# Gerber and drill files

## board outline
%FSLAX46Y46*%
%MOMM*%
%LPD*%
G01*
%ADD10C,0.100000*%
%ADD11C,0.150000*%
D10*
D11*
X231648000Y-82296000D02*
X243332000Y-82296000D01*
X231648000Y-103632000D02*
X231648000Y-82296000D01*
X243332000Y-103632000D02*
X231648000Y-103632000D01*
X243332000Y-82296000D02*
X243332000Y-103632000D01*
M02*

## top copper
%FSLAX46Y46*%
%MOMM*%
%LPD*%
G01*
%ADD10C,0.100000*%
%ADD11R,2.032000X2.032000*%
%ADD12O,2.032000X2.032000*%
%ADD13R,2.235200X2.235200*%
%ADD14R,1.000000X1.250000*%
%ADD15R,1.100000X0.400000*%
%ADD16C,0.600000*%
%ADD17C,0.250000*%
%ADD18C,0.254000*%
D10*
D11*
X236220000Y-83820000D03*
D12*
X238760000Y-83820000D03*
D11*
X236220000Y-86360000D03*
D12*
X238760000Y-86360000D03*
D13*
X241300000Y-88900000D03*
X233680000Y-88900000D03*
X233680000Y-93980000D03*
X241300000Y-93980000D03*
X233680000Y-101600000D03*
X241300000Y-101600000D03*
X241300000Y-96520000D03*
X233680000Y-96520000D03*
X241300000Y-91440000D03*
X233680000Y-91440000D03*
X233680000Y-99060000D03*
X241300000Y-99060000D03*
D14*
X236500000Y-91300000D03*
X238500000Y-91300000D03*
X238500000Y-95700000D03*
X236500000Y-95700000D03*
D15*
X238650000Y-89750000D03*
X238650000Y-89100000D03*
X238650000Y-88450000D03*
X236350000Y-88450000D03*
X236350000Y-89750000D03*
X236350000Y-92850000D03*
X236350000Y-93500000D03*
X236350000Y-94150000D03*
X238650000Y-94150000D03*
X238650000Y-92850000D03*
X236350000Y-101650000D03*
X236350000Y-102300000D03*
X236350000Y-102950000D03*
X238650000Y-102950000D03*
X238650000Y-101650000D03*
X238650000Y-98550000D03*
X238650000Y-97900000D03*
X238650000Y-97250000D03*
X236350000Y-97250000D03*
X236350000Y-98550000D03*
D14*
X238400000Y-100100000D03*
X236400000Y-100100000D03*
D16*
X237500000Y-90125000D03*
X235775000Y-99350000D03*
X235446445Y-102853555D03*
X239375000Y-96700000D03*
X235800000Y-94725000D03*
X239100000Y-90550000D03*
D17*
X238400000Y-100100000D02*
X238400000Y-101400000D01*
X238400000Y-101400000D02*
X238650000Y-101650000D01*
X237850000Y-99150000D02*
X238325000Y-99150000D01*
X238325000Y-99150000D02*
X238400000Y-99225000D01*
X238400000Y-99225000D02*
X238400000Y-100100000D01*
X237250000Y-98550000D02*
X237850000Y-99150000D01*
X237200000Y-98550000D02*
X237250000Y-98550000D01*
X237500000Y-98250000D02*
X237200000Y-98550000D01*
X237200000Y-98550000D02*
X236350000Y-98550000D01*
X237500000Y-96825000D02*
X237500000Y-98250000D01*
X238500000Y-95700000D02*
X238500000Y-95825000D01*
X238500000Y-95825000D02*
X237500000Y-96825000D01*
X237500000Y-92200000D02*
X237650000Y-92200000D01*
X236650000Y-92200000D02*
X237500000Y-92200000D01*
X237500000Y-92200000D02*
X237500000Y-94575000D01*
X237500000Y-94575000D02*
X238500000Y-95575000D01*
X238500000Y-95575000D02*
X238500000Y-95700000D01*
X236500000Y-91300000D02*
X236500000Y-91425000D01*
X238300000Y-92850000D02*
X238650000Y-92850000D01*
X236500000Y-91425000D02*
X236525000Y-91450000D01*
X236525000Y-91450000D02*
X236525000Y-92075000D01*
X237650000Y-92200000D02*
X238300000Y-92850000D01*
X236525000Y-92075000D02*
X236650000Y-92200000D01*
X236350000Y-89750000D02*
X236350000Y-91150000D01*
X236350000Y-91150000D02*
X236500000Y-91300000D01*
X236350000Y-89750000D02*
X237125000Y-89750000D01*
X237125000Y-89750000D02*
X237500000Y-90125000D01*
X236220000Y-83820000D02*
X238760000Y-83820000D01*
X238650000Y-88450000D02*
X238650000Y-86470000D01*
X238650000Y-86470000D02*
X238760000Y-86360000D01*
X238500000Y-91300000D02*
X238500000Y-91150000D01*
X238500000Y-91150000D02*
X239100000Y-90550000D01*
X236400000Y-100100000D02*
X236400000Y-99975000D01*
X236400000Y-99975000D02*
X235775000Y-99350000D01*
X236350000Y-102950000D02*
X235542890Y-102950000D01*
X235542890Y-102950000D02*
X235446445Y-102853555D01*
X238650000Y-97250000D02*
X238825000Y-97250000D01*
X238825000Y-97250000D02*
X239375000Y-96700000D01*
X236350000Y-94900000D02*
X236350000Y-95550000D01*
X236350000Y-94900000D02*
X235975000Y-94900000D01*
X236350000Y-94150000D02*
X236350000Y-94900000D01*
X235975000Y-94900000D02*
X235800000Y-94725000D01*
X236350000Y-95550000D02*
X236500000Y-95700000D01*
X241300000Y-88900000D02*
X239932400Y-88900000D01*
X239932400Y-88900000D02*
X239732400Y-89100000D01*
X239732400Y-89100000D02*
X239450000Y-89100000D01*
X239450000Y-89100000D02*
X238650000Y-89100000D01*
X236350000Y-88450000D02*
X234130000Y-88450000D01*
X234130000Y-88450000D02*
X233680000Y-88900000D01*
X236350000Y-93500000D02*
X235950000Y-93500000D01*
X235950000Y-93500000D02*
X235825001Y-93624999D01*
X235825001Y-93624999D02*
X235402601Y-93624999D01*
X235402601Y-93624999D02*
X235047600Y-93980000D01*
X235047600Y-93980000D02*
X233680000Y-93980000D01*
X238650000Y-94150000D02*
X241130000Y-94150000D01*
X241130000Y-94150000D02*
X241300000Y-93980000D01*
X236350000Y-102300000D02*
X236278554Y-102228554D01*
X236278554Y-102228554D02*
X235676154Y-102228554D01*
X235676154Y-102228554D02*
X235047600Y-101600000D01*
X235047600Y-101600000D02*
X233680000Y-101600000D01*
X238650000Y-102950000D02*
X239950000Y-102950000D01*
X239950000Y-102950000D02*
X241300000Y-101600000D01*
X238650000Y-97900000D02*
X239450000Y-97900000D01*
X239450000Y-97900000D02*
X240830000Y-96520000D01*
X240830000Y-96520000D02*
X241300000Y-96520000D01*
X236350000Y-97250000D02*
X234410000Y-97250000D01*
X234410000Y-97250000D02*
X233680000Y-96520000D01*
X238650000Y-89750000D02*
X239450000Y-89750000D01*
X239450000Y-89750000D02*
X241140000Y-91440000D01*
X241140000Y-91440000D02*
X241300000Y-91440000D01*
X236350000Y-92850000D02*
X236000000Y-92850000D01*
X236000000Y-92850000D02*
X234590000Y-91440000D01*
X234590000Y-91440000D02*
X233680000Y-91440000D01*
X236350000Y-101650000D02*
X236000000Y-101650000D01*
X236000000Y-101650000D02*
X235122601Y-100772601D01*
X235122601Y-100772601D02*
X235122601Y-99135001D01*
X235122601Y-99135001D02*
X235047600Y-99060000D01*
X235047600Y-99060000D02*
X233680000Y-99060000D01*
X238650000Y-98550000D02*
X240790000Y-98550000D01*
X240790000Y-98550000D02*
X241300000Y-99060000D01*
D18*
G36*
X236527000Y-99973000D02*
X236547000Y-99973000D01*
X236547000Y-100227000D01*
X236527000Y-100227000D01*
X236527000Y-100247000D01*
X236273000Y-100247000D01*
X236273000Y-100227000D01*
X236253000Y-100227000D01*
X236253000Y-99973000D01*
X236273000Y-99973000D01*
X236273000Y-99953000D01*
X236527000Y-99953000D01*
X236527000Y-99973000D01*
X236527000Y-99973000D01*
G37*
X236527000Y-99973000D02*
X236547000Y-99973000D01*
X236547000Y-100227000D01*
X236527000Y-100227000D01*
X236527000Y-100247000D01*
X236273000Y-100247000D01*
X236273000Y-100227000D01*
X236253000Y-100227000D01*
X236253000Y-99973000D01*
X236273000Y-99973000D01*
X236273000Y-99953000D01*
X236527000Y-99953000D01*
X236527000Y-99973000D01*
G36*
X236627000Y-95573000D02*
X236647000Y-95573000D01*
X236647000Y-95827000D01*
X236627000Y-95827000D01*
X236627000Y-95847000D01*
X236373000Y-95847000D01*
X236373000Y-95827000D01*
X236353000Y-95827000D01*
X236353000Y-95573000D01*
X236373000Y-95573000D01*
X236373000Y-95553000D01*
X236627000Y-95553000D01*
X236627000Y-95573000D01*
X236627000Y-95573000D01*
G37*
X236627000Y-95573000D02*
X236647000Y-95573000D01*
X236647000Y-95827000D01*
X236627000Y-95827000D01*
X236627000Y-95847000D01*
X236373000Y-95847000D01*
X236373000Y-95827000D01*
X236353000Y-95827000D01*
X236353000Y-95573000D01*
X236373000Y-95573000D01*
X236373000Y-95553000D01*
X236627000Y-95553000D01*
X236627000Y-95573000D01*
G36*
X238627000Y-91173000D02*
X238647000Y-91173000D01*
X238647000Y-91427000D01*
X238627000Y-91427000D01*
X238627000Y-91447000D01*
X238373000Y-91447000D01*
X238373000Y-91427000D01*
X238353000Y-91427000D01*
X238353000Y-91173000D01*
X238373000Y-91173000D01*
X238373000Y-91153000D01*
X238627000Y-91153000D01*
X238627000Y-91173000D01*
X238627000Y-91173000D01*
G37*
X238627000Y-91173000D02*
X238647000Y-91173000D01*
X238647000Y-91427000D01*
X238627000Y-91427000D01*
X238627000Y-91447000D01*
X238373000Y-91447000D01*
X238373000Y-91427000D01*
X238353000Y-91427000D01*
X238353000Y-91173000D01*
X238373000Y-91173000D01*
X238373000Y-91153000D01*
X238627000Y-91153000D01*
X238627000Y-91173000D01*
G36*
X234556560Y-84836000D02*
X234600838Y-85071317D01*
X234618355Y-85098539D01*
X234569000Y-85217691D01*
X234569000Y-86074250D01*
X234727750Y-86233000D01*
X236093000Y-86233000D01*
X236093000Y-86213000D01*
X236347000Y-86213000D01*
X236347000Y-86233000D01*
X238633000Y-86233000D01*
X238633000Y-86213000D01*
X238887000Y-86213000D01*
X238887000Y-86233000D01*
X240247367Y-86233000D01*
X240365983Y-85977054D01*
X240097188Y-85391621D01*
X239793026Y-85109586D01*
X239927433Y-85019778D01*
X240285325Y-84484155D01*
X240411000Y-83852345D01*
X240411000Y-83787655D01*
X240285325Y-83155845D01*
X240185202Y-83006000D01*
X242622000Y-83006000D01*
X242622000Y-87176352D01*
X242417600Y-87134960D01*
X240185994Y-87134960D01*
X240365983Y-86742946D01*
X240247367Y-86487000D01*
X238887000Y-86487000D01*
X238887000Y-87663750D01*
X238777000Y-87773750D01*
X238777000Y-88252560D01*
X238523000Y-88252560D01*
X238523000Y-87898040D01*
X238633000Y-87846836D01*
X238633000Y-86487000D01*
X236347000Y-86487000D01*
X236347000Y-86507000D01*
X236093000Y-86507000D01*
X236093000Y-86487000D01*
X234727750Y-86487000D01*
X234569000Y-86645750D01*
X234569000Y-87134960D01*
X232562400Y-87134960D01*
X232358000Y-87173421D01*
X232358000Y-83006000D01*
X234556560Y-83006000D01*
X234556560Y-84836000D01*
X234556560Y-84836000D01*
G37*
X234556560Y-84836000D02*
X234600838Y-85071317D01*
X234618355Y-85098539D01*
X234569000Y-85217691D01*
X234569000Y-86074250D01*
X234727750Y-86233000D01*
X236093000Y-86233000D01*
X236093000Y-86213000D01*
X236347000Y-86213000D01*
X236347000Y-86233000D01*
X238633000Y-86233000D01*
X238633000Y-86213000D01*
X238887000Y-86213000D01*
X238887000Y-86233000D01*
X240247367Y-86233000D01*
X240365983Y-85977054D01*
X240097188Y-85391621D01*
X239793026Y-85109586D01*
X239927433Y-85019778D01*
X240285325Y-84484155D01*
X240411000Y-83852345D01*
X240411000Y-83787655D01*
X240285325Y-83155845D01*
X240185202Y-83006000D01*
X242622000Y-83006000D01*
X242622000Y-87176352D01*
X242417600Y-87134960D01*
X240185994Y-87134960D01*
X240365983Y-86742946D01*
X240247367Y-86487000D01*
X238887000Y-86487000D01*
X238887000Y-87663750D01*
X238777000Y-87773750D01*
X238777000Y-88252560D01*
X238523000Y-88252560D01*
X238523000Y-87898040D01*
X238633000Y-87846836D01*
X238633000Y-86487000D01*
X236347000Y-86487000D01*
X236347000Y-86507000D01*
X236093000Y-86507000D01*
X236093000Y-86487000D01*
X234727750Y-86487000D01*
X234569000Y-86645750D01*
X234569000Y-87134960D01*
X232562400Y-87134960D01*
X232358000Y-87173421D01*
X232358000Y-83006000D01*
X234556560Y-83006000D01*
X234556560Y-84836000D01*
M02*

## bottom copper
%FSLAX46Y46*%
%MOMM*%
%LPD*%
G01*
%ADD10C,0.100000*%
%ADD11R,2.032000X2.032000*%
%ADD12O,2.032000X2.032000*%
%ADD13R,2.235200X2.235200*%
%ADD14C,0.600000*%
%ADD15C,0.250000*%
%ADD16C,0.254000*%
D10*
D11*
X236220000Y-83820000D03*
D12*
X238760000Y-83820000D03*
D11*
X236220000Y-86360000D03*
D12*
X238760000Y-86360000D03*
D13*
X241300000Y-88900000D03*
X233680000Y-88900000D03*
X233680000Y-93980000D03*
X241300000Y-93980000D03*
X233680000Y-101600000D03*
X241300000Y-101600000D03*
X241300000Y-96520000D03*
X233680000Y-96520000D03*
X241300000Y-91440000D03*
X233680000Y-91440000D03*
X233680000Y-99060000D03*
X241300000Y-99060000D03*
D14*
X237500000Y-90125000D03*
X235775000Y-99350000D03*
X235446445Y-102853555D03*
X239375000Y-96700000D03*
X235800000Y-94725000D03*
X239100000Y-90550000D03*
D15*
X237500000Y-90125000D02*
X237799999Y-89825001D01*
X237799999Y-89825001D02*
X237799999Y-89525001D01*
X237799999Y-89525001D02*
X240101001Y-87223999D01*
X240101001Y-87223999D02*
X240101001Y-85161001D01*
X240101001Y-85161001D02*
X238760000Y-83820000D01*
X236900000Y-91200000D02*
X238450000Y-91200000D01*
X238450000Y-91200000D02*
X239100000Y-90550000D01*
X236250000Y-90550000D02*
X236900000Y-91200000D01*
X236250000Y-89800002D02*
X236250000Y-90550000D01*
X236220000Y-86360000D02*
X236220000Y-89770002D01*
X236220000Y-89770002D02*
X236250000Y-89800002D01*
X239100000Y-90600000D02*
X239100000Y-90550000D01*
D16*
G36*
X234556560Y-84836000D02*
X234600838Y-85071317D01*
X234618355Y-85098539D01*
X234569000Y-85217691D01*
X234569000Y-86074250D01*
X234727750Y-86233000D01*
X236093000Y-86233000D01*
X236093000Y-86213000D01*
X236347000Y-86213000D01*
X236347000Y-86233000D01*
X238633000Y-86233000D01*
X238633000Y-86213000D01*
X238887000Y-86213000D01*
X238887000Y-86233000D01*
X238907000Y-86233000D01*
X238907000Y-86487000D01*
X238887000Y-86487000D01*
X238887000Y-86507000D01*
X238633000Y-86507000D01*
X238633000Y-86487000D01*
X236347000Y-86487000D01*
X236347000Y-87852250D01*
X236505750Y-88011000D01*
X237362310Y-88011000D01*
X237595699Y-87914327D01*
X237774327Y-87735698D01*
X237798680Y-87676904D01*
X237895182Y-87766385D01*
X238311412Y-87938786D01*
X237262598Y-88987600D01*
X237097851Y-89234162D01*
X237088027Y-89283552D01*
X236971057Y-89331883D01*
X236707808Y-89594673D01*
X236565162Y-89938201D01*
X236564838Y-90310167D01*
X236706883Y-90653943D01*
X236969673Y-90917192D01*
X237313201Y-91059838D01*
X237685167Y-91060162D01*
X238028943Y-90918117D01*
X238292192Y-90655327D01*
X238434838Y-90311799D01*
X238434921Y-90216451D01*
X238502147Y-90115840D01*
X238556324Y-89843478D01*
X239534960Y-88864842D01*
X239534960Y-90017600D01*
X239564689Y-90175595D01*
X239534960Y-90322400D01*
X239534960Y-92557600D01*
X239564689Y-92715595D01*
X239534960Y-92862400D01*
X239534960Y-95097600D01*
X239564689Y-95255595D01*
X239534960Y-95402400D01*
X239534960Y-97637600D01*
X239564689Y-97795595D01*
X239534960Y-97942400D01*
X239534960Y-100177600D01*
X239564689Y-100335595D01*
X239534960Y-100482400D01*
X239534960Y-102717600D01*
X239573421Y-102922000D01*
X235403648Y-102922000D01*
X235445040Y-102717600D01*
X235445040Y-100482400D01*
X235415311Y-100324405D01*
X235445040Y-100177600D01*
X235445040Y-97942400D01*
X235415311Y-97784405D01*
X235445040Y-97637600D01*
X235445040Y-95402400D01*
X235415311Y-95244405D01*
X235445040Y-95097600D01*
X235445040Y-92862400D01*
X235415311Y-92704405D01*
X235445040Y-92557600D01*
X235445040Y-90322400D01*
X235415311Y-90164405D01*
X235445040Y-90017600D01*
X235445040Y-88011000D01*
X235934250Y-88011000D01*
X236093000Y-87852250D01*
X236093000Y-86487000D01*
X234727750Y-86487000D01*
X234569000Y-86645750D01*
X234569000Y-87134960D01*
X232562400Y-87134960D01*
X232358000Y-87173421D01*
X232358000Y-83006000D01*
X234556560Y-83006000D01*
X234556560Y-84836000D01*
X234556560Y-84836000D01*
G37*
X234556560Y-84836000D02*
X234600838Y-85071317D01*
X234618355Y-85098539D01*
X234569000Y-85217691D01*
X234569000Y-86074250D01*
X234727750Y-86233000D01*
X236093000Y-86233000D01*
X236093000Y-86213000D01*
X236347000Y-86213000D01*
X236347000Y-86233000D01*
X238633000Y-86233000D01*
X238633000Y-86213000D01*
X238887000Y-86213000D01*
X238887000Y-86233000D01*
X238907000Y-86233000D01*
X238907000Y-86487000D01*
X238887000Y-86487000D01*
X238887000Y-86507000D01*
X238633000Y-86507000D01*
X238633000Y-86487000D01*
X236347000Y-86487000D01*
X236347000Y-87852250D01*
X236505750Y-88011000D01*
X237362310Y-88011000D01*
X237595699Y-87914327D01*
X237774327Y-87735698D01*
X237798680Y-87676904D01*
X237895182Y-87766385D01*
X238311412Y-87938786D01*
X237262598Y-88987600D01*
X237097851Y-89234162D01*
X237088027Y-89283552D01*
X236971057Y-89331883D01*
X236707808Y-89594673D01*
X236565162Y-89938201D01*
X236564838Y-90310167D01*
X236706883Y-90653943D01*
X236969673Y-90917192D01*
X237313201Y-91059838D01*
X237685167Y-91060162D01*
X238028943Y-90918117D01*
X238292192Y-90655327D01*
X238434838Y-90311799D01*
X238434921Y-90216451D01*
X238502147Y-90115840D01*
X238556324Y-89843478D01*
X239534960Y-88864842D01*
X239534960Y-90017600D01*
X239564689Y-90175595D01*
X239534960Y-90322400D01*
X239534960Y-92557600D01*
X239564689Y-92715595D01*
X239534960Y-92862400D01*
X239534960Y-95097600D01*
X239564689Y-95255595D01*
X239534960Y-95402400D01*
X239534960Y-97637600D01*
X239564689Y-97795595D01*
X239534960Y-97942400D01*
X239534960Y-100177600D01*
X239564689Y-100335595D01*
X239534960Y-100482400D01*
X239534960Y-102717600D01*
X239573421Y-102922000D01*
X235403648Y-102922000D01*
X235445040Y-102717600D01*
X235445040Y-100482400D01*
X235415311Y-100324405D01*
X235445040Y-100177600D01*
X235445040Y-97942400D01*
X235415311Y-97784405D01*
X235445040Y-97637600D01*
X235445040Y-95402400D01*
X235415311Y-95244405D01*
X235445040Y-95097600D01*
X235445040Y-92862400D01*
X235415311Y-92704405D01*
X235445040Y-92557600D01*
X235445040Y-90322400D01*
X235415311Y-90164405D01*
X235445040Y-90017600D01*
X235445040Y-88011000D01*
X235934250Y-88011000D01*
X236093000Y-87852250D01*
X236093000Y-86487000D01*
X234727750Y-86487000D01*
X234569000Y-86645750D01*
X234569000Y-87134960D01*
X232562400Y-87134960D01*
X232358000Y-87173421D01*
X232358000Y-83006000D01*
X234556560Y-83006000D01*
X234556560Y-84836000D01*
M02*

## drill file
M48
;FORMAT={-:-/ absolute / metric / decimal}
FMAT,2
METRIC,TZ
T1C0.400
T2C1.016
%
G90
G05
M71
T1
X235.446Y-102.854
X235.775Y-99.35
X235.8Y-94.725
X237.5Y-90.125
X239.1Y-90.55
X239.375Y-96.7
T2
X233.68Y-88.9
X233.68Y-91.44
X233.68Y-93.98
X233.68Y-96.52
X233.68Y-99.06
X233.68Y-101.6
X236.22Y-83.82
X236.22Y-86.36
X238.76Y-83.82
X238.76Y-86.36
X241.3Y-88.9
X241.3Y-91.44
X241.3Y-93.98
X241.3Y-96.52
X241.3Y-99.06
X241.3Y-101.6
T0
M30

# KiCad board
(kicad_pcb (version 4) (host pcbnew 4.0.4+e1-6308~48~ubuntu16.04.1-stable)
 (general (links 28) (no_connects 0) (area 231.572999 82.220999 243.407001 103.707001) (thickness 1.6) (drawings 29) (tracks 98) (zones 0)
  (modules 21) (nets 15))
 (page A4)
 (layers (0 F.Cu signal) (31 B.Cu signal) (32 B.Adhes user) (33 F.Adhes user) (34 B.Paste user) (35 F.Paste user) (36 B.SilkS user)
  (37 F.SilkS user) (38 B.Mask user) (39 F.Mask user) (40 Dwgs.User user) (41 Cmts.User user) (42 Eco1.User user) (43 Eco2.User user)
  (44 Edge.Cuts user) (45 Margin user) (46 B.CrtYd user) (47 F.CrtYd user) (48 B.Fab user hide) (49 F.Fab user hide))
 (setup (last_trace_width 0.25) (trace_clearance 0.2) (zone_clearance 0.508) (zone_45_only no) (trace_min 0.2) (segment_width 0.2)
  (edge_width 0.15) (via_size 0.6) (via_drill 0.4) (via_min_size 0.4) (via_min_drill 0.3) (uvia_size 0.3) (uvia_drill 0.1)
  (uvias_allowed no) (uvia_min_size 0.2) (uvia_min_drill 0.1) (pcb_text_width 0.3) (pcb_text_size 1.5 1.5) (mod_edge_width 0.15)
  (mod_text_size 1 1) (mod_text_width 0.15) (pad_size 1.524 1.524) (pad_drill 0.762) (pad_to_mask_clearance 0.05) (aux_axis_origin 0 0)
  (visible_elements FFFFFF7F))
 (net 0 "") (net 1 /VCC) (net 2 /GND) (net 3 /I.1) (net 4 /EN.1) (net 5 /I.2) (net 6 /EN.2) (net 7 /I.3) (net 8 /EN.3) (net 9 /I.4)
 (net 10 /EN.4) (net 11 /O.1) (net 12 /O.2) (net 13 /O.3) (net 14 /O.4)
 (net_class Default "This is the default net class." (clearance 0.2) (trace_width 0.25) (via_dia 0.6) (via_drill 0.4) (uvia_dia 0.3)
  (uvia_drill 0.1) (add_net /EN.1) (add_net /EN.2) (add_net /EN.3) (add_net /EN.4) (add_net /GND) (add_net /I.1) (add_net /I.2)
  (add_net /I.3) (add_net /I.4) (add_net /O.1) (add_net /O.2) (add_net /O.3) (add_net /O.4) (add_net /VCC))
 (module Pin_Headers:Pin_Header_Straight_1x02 (layer F.Cu) (at 236.22 83.82 90)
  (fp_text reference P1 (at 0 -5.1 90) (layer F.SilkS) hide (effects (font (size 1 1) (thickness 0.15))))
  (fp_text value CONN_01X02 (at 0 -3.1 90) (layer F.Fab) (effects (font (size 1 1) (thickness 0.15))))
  (pad 1 thru_hole rect (at 0 0 90) (size 2.032 2.032) (drill 1.016) (layers *.Cu *.Mask F.SilkS) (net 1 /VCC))
  (pad 2 thru_hole oval (at 0 2.54 90) (size 2.032 2.032) (drill 1.016) (layers *.Cu *.Mask F.SilkS) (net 1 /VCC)))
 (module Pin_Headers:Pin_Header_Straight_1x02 (layer F.Cu) (at 236.22 86.36 90)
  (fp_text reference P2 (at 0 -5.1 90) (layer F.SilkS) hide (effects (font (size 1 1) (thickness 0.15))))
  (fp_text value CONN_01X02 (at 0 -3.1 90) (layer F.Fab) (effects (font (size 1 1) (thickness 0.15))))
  (pad 1 thru_hole rect (at 0 0 90) (size 2.032 2.032) (drill 1.016) (layers *.Cu *.Mask F.SilkS) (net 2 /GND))
  (pad 2 thru_hole oval (at 0 2.54 90) (size 2.032 2.032) (drill 1.016) (layers *.Cu *.Mask F.SilkS) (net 2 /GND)))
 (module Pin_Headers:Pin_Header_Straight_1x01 (layer F.Cu) (at 241.3 88.9 270)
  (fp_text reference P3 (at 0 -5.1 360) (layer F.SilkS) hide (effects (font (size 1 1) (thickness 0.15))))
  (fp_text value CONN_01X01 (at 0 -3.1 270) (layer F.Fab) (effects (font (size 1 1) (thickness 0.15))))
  (pad 1 thru_hole rect (at 0 0 270) (size 2.2352 2.2352) (drill 1.016) (layers *.Cu *.Mask F.SilkS) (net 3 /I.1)))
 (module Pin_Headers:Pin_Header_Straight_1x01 (layer F.Cu) (at 233.68 88.9 90)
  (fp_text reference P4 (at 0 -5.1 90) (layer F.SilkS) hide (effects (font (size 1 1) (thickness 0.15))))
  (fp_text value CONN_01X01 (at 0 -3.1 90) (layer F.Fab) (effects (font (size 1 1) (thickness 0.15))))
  (pad 1 thru_hole rect (at 0 0 90) (size 2.2352 2.2352) (drill 1.016) (layers *.Cu *.Mask F.SilkS) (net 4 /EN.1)))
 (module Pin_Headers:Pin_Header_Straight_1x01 (layer F.Cu) (at 233.68 93.98 90)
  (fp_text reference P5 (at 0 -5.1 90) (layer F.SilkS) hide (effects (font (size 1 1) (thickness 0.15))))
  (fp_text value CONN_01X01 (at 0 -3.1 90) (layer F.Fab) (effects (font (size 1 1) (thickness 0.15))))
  (pad 1 thru_hole rect (at 0 0 90) (size 2.2352 2.2352) (drill 1.016) (layers *.Cu *.Mask F.SilkS) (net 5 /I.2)))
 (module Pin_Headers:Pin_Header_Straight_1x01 (layer F.Cu) (at 241.3 93.98 270)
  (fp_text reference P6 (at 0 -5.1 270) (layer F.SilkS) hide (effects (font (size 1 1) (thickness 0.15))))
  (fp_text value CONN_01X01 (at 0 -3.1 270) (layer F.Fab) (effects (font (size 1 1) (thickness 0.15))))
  (pad 1 thru_hole rect (at 0 0 270) (size 2.2352 2.2352) (drill 1.016) (layers *.Cu *.Mask F.SilkS) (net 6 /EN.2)))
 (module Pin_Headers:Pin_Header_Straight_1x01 (layer F.Cu) (at 233.68 101.6 90)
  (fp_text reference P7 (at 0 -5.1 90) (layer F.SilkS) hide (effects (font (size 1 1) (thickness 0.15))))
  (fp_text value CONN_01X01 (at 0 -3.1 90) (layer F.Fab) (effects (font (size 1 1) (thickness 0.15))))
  (pad 1 thru_hole rect (at 0 0 90) (size 2.2352 2.2352) (drill 1.016) (layers *.Cu *.Mask F.SilkS) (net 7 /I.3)))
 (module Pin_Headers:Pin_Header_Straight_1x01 (layer F.Cu) (at 241.3 101.6 270)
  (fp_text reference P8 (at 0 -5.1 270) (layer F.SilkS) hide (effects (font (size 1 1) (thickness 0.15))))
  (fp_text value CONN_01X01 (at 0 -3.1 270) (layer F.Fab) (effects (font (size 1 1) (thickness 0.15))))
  (pad 1 thru_hole rect (at 0 0 270) (size 2.2352 2.2352) (drill 1.016) (layers *.Cu *.Mask F.SilkS) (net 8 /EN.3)))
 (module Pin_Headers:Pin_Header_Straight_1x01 (layer F.Cu) (at 241.3 96.52 270)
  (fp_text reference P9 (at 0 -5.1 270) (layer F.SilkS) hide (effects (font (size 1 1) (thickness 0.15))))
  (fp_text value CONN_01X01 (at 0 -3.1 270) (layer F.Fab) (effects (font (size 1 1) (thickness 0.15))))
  (pad 1 thru_hole rect (at 0 0 270) (size 2.2352 2.2352) (drill 1.016) (layers *.Cu *.Mask F.SilkS) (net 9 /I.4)))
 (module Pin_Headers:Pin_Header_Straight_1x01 (layer F.Cu) (at 233.68 96.52 90)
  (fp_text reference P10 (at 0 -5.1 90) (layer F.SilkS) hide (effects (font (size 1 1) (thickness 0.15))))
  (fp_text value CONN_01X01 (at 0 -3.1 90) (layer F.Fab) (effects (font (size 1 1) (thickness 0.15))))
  (pad 1 thru_hole rect (at 0 0 90) (size 2.2352 2.2352) (drill 1.016) (layers *.Cu *.Mask F.SilkS) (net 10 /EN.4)))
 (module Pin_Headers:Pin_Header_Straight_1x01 (layer F.Cu) (at 241.3 91.44 270)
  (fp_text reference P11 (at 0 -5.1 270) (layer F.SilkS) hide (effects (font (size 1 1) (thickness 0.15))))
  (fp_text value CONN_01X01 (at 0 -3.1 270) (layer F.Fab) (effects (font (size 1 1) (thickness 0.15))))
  (pad 1 thru_hole rect (at 0 0 270) (size 2.2352 2.2352) (drill 1.016) (layers *.Cu *.Mask F.SilkS) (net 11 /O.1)))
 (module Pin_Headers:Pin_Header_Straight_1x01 (layer F.Cu) (at 233.68 91.44 90)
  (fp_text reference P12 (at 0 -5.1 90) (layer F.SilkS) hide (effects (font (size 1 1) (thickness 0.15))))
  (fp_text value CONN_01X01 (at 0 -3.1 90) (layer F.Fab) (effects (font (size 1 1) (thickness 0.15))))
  (pad 1 thru_hole rect (at 0 0 90) (size 2.2352 2.2352) (drill 1.016) (layers *.Cu *.Mask F.SilkS) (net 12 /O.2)))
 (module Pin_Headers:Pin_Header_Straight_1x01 (layer F.Cu) (at 233.68 99.06 90)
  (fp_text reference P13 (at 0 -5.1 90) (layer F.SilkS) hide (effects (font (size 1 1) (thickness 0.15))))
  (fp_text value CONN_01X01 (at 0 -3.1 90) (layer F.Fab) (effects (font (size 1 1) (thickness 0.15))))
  (pad 1 thru_hole rect (at 0 0 90) (size 2.2352 2.2352) (drill 1.016) (layers *.Cu *.Mask F.SilkS) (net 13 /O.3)))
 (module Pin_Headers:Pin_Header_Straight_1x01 (layer F.Cu) (at 241.3 99.06 270)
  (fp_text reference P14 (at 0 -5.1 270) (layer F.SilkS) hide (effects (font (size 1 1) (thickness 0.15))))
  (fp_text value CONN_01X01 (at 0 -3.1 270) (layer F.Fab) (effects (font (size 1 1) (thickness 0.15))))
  (pad 1 thru_hole rect (at 0 0 270) (size 2.2352 2.2352) (drill 1.016) (layers *.Cu *.Mask F.SilkS) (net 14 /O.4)))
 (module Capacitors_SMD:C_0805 (layer F.Cu) (at 237.5 91.3)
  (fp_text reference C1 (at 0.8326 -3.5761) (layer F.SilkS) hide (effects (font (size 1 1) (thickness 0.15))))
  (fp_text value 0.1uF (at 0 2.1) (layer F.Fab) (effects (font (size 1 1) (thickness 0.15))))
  (pad 1 smd rect (at -1 0) (size 1 1.25) (layers F.Cu F.Paste F.Mask) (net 1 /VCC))
  (pad 2 smd rect (at 1 0) (size 1 1.25) (layers F.Cu F.Paste F.Mask) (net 2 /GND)))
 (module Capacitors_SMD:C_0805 (layer F.Cu) (at 237.5 95.7 180)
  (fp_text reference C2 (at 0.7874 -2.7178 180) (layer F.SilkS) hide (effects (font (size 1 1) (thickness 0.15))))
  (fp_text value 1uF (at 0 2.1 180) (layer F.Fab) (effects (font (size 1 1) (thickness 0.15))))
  (pad 1 smd rect (at -1 0 180) (size 1 1.25) (layers F.Cu F.Paste F.Mask) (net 1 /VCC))
  (pad 2 smd rect (at 1 0 180) (size 1 1.25) (layers F.Cu F.Paste F.Mask) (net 2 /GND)))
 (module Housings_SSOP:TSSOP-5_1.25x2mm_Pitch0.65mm (layer F.Cu) (at 237.5 89.1 180)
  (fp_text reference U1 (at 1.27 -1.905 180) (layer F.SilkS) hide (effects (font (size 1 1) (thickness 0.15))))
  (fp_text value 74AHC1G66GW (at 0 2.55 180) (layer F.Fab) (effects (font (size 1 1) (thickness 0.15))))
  (pad 1 smd rect (at -1.15 -0.65 180) (size 1.1 0.4) (layers F.Cu F.Paste F.Mask) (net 11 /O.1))
  (pad 2 smd rect (at -1.15 0 180) (size 1.1 0.4) (layers F.Cu F.Paste F.Mask) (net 3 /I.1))
  (pad 3 smd rect (at -1.15 0.65 180) (size 1.1 0.4) (layers F.Cu F.Paste F.Mask) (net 2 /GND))
  (pad 4 smd rect (at 1.15 0.65 180) (size 1.1 0.4) (layers F.Cu F.Paste F.Mask) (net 4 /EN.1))
  (pad 5 smd rect (at 1.15 -0.65) (size 1.1 0.4) (layers F.Cu F.Paste F.Mask) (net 1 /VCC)))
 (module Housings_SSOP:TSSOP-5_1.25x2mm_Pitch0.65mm (layer F.Cu) (at 237.5 93.5)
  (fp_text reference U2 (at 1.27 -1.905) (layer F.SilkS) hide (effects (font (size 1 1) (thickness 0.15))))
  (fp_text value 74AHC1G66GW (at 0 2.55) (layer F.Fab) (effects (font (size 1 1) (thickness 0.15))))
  (pad 1 smd rect (at -1.15 -0.65) (size 1.1 0.4) (layers F.Cu F.Paste F.Mask) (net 12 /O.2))
  (pad 2 smd rect (at -1.15 0) (size 1.1 0.4) (layers F.Cu F.Paste F.Mask) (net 5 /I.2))
  (pad 3 smd rect (at -1.15 0.65) (size 1.1 0.4) (layers F.Cu F.Paste F.Mask) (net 2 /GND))
  (pad 4 smd rect (at 1.15 0.65) (size 1.1 0.4) (layers F.Cu F.Paste F.Mask) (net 6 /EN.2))
  (pad 5 smd rect (at 1.15 -0.65 180) (size 1.1 0.4) (layers F.Cu F.Paste F.Mask) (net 1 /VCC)))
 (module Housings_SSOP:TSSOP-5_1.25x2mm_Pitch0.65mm (layer F.Cu) (at 237.5 102.3)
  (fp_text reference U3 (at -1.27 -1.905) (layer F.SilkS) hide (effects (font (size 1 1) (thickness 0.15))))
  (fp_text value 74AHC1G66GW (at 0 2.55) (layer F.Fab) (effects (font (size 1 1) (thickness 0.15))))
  (pad 1 smd rect (at -1.15 -0.65) (size 1.1 0.4) (layers F.Cu F.Paste F.Mask) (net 13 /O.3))
  (pad 2 smd rect (at -1.15 0) (size 1.1 0.4) (layers F.Cu F.Paste F.Mask) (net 7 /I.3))
  (pad 3 smd rect (at -1.15 0.65) (size 1.1 0.4) (layers F.Cu F.Paste F.Mask) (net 2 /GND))
  (pad 4 smd rect (at 1.15 0.65) (size 1.1 0.4) (layers F.Cu F.Paste F.Mask) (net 8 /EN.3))
  (pad 5 smd rect (at 1.15 -0.65 180) (size 1.1 0.4) (layers F.Cu F.Paste F.Mask) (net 1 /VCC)))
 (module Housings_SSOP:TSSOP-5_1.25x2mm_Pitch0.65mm (layer F.Cu) (at 237.5 97.9 180)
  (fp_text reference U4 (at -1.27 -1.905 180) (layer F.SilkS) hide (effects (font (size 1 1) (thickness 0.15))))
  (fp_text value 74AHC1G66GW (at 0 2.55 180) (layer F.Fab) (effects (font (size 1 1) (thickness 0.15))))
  (pad 1 smd rect (at -1.15 -0.65 180) (size 1.1 0.4) (layers F.Cu F.Paste F.Mask) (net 14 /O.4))
  (pad 2 smd rect (at -1.15 0 180) (size 1.1 0.4) (layers F.Cu F.Paste F.Mask) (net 9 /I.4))
  (pad 3 smd rect (at -1.15 0.65 180) (size 1.1 0.4) (layers F.Cu F.Paste F.Mask) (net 2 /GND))
  (pad 4 smd rect (at 1.15 0.65 180) (size 1.1 0.4) (layers F.Cu F.Paste F.Mask) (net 10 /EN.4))
  (pad 5 smd rect (at 1.15 -0.65) (size 1.1 0.4) (layers F.Cu F.Paste F.Mask) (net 1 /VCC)))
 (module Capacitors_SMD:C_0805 (layer F.Cu) (at 237.4 100.1 180)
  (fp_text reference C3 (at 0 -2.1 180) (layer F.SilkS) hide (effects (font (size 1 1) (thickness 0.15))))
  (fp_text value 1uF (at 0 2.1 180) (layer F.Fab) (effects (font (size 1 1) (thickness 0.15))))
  (pad 1 smd rect (at -1 0 180) (size 1 1.25) (layers F.Cu F.Paste F.Mask) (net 1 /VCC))
  (pad 2 smd rect (at 1 0 180) (size 1 1.25) (layers F.Cu F.Paste F.Mask) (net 2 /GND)))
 (gr_line (start 231.648 82.296) (end 243.332 82.296) (layer Edge.Cuts) (width 0.15))
 (gr_line (start 231.648 103.632) (end 231.648 82.296) (layer Edge.Cuts) (width 0.15))
 (gr_line (start 243.332 103.632) (end 231.648 103.632) (layer Edge.Cuts) (width 0.15))
 (gr_line (start 243.332 82.296) (end 243.332 103.632) (layer Edge.Cuts) (width 0.15))
 (segment (start 238.4 100.1) (end 238.4 101.4) (width 0.25) (layer F.Cu) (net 1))
 (segment (start 238.4 101.4) (end 238.65 101.65) (width 0.25) (layer F.Cu) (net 1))
 (segment (start 237.85 99.15) (end 238.325 99.15) (width 0.25) (layer F.Cu) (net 1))
 (segment (start 238.325 99.15) (end 238.4 99.225) (width 0.25) (layer F.Cu) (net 1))
 (segment (start 238.4 99.225) (end 238.4 100.1) (width 0.25) (layer F.Cu) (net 1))
 (segment (start 237.25 98.55) (end 237.85 99.15) (width 0.25) (layer F.Cu) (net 1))
 (segment (start 237.2 98.55) (end 237.25 98.55) (width 0.25) (layer F.Cu) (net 1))
 (segment (start 237.5 98.25) (end 237.2 98.55) (width 0.25) (layer F.Cu) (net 1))
 (segment (start 237.2 98.55) (end 236.35 98.55) (width 0.25) (layer F.Cu) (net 1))
 (segment (start 237.5 96.825) (end 237.5 98.25) (width 0.25) (layer F.Cu) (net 1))
 (segment (start 238.5 95.7) (end 238.5 95.825) (width 0.25) (layer F.Cu) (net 1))
 (segment (start 238.5 95.825) (end 237.5 96.825) (width 0.25) (layer F.Cu) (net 1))
 (segment (start 237.5 92.2) (end 237.65 92.2) (width 0.25) (layer F.Cu) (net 1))
 (segment (start 236.65 92.2) (end 237.5 92.2) (width 0.25) (layer F.Cu) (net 1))
 (segment (start 237.5 92.2) (end 237.5 94.575) (width 0.25) (layer F.Cu) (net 1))
 (segment (start 237.5 94.575) (end 238.5 95.575) (width 0.25) (layer F.Cu) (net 1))
 (segment (start 238.5 95.575) (end 238.5 95.7) (width 0.25) (layer F.Cu) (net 1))
 (segment (start 236.5 91.3) (end 236.5 91.425) (width 0.25) (layer F.Cu) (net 1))
 (segment (start 238.3 92.85) (end 238.65 92.85) (width 0.25) (layer F.Cu) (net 1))
 (segment (start 236.5 91.425) (end 236.525 91.45) (width 0.25) (layer F.Cu) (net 1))
 (segment (start 236.525 91.45) (end 236.525 92.075) (width 0.25) (layer F.Cu) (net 1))
 (segment (start 237.65 92.2) (end 238.3 92.85) (width 0.25) (layer F.Cu) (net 1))
 (segment (start 236.525 92.075) (end 236.65 92.2) (width 0.25) (layer F.Cu) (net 1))
 (segment (start 236.35 89.75) (end 236.35 91.15) (width 0.25) (layer F.Cu) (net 1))
 (segment (start 236.35 91.15) (end 236.5 91.3) (width 0.25) (layer F.Cu) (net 1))
 (segment (start 237.5 90.125) (end 237.799999 89.825001) (width 0.25) (layer B.Cu) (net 1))
 (segment (start 237.799999 89.825001) (end 237.799999 89.525001) (width 0.25) (layer B.Cu) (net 1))
 (segment (start 237.799999 89.525001) (end 240.101001 87.223999) (width 0.25) (layer B.Cu) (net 1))
 (segment (start 240.101001 87.223999) (end 240.101001 85.161001) (width 0.25) (layer B.Cu) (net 1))
 (segment (start 240.101001 85.161001) (end 238.76 83.82) (width 0.25) (layer B.Cu) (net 1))
 (segment (start 236.35 89.75) (end 237.125 89.75) (width 0.25) (layer F.Cu) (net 1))
 (segment (start 237.125 89.75) (end 237.5 90.125) (width 0.25) (layer F.Cu) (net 1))
 (via (at 237.5 90.125) (size 0.6) (drill 0.4) (layers F.Cu B.Cu) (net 1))
 (segment (start 236.22 83.82) (end 238.76 83.82) (width 0.25) (layer F.Cu) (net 1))
 (segment (start 238.65 88.45) (end 238.65 86.47) (width 0.25) (layer F.Cu) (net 2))
 (segment (start 238.65 86.47) (end 238.76 86.36) (width 0.25) (layer F.Cu) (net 2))
 (segment (start 238.5 91.3) (end 238.5 91.15) (width 0.25) (layer F.Cu) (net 2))
 (segment (start 238.5 91.15) (end 239.1 90.55) (width 0.25) (layer F.Cu) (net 2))
 (segment (start 236.9 91.2) (end 238.45 91.2) (width 0.25) (layer B.Cu) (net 2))
 (segment (start 238.45 91.2) (end 239.1 90.55) (width 0.25) (layer B.Cu) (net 2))
 (segment (start 236.25 90.55) (end 236.9 91.2) (width 0.25) (layer B.Cu) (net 2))
 (segment (start 236.25 89.800002) (end 236.25 90.55) (width 0.25) (layer B.Cu) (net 2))
 (segment (start 236.22 86.36) (end 236.22 89.770002) (width 0.25) (layer B.Cu) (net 2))
 (segment (start 236.22 89.770002) (end 236.25 89.800002) (width 0.25) (layer B.Cu) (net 2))
 (segment (start 239.1 90.6) (end 239.1 90.55) (width 0.25) (layer B.Cu) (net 2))
 (segment (start 236.4 100.1) (end 236.4 99.975) (width 0.25) (layer F.Cu) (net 2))
 (segment (start 236.4 99.975) (end 235.775 99.35) (width 0.25) (layer F.Cu) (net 2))
 (via (at 235.775 99.35) (size 0.6) (drill 0.4) (layers F.Cu B.Cu) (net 2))
 (segment (start 236.35 102.95) (end 235.54289 102.95) (width 0.25) (layer F.Cu) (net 2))
 (segment (start 235.54289 102.95) (end 235.446445 102.853555) (width 0.25) (layer F.Cu) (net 2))
 (via (at 235.446445 102.853555) (size 0.6) (drill 0.4) (layers F.Cu B.Cu) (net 2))
 (segment (start 238.65 97.25) (end 238.825 97.25) (width 0.25) (layer F.Cu) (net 2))
 (segment (start 238.825 97.25) (end 239.375 96.7) (width 0.25) (layer F.Cu) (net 2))
 (via (at 239.375 96.7) (size 0.6) (drill 0.4) (layers F.Cu B.Cu) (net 2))
 (segment (start 236.35 94.9) (end 236.35 95.55) (width 0.25) (layer F.Cu) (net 2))
 (segment (start 236.35 94.9) (end 235.975 94.9) (width 0.25) (layer F.Cu) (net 2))
 (segment (start 236.35 94.15) (end 236.35 94.9) (width 0.25) (layer F.Cu) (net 2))
 (segment (start 235.975 94.9) (end 235.8 94.725) (width 0.25) (layer F.Cu) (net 2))
 (via (at 235.8 94.725) (size 0.6) (drill 0.4) (layers F.Cu B.Cu) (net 2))
 (segment (start 236.35 95.55) (end 236.5 95.7) (width 0.25) (layer F.Cu) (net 2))
 (via (at 239.1 90.55) (size 0.6) (drill 0.4) (layers F.Cu B.Cu) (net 2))
 (segment (start 241.3 88.9) (end 239.9324 88.9) (width 0.25) (layer F.Cu) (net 3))
 (segment (start 239.9324 88.9) (end 239.7324 89.1) (width 0.25) (layer F.Cu) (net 3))
 (segment (start 239.7324 89.1) (end 239.45 89.1) (width 0.25) (layer F.Cu) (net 3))
 (segment (start 239.45 89.1) (end 238.65 89.1) (width 0.25) (layer F.Cu) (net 3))
 (segment (start 236.35 88.45) (end 234.13 88.45) (width 0.25) (layer F.Cu) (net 4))
 (segment (start 234.13 88.45) (end 233.68 88.9) (width 0.25) (layer F.Cu) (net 4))
 (segment (start 236.35 93.5) (end 235.95 93.5) (width 0.25) (layer F.Cu) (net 5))
 (segment (start 235.95 93.5) (end 235.825001 93.624999) (width 0.25) (layer F.Cu) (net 5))
 (segment (start 235.825001 93.624999) (end 235.402601 93.624999) (width 0.25) (layer F.Cu) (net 5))
 (segment (start 235.402601 93.624999) (end 235.0476 93.98) (width 0.25) (layer F.Cu) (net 5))
 (segment (start 235.0476 93.98) (end 233.68 93.98) (width 0.25) (layer F.Cu) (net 5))
 (segment (start 238.65 94.15) (end 241.13 94.15) (width 0.25) (layer F.Cu) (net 6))
 (segment (start 241.13 94.15) (end 241.3 93.98) (width 0.25) (layer F.Cu) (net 6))
 (segment (start 236.35 102.3) (end 236.278554 102.228554) (width 0.25) (layer F.Cu) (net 7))
 (segment (start 236.278554 102.228554) (end 235.676154 102.228554) (width 0.25) (layer F.Cu) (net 7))
 (segment (start 235.676154 102.228554) (end 235.0476 101.6) (width 0.25) (layer F.Cu) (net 7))
 (segment (start 235.0476 101.6) (end 233.68 101.6) (width 0.25) (layer F.Cu) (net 7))
 (segment (start 238.65 102.95) (end 239.95 102.95) (width 0.25) (layer F.Cu) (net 8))
 (segment (start 239.95 102.95) (end 241.3 101.6) (width 0.25) (layer F.Cu) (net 8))
 (segment (start 238.65 97.9) (end 239.45 97.9) (width 0.25) (layer F.Cu) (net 9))
 (segment (start 239.45 97.9) (end 240.83 96.52) (width 0.25) (layer F.Cu) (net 9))
 (segment (start 240.83 96.52) (end 241.3 96.52) (width 0.25) (layer F.Cu) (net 9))
 (segment (start 236.35 97.25) (end 234.41 97.25) (width 0.25) (layer F.Cu) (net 10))
 (segment (start 234.41 97.25) (end 233.68 96.52) (width 0.25) (layer F.Cu) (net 10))
 (segment (start 238.65 89.75) (end 239.45 89.75) (width 0.25) (layer F.Cu) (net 11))
 (segment (start 239.45 89.75) (end 241.14 91.44) (width 0.25) (layer F.Cu) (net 11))
 (segment (start 241.14 91.44) (end 241.3 91.44) (width 0.25) (layer F.Cu) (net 11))
 (segment (start 236.35 92.85) (end 236 92.85) (width 0.25) (layer F.Cu) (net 12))
 (segment (start 236 92.85) (end 234.59 91.44) (width 0.25) (layer F.Cu) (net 12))
 (segment (start 234.59 91.44) (end 233.68 91.44) (width 0.25) (layer F.Cu) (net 12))
 (segment (start 236.35 101.65) (end 236 101.65) (width 0.25) (layer F.Cu) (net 13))
 (segment (start 236 101.65) (end 235.122601 100.772601) (width 0.25) (layer F.Cu) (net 13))
 (segment (start 235.122601 100.772601) (end 235.122601 99.135001) (width 0.25) (layer F.Cu) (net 13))
 (segment (start 235.122601 99.135001) (end 235.0476 99.06) (width 0.25) (layer F.Cu) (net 13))
 (segment (start 235.0476 99.06) (end 233.68 99.06) (width 0.25) (layer F.Cu) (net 13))
 (segment (start 238.65 98.55) (end 240.79 98.55) (width 0.25) (layer F.Cu) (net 14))
 (segment (start 240.79 98.55) (end 241.3 99.06) (width 0.25) (layer F.Cu) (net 14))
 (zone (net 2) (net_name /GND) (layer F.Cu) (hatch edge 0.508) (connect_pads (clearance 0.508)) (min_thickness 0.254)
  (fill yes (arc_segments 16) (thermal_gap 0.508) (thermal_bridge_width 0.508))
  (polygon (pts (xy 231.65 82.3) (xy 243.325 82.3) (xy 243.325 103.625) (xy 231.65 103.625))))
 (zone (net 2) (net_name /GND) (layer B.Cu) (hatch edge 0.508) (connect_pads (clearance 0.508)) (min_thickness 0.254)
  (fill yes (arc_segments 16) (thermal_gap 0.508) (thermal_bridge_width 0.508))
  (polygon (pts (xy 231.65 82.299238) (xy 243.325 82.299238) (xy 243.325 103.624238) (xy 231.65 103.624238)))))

